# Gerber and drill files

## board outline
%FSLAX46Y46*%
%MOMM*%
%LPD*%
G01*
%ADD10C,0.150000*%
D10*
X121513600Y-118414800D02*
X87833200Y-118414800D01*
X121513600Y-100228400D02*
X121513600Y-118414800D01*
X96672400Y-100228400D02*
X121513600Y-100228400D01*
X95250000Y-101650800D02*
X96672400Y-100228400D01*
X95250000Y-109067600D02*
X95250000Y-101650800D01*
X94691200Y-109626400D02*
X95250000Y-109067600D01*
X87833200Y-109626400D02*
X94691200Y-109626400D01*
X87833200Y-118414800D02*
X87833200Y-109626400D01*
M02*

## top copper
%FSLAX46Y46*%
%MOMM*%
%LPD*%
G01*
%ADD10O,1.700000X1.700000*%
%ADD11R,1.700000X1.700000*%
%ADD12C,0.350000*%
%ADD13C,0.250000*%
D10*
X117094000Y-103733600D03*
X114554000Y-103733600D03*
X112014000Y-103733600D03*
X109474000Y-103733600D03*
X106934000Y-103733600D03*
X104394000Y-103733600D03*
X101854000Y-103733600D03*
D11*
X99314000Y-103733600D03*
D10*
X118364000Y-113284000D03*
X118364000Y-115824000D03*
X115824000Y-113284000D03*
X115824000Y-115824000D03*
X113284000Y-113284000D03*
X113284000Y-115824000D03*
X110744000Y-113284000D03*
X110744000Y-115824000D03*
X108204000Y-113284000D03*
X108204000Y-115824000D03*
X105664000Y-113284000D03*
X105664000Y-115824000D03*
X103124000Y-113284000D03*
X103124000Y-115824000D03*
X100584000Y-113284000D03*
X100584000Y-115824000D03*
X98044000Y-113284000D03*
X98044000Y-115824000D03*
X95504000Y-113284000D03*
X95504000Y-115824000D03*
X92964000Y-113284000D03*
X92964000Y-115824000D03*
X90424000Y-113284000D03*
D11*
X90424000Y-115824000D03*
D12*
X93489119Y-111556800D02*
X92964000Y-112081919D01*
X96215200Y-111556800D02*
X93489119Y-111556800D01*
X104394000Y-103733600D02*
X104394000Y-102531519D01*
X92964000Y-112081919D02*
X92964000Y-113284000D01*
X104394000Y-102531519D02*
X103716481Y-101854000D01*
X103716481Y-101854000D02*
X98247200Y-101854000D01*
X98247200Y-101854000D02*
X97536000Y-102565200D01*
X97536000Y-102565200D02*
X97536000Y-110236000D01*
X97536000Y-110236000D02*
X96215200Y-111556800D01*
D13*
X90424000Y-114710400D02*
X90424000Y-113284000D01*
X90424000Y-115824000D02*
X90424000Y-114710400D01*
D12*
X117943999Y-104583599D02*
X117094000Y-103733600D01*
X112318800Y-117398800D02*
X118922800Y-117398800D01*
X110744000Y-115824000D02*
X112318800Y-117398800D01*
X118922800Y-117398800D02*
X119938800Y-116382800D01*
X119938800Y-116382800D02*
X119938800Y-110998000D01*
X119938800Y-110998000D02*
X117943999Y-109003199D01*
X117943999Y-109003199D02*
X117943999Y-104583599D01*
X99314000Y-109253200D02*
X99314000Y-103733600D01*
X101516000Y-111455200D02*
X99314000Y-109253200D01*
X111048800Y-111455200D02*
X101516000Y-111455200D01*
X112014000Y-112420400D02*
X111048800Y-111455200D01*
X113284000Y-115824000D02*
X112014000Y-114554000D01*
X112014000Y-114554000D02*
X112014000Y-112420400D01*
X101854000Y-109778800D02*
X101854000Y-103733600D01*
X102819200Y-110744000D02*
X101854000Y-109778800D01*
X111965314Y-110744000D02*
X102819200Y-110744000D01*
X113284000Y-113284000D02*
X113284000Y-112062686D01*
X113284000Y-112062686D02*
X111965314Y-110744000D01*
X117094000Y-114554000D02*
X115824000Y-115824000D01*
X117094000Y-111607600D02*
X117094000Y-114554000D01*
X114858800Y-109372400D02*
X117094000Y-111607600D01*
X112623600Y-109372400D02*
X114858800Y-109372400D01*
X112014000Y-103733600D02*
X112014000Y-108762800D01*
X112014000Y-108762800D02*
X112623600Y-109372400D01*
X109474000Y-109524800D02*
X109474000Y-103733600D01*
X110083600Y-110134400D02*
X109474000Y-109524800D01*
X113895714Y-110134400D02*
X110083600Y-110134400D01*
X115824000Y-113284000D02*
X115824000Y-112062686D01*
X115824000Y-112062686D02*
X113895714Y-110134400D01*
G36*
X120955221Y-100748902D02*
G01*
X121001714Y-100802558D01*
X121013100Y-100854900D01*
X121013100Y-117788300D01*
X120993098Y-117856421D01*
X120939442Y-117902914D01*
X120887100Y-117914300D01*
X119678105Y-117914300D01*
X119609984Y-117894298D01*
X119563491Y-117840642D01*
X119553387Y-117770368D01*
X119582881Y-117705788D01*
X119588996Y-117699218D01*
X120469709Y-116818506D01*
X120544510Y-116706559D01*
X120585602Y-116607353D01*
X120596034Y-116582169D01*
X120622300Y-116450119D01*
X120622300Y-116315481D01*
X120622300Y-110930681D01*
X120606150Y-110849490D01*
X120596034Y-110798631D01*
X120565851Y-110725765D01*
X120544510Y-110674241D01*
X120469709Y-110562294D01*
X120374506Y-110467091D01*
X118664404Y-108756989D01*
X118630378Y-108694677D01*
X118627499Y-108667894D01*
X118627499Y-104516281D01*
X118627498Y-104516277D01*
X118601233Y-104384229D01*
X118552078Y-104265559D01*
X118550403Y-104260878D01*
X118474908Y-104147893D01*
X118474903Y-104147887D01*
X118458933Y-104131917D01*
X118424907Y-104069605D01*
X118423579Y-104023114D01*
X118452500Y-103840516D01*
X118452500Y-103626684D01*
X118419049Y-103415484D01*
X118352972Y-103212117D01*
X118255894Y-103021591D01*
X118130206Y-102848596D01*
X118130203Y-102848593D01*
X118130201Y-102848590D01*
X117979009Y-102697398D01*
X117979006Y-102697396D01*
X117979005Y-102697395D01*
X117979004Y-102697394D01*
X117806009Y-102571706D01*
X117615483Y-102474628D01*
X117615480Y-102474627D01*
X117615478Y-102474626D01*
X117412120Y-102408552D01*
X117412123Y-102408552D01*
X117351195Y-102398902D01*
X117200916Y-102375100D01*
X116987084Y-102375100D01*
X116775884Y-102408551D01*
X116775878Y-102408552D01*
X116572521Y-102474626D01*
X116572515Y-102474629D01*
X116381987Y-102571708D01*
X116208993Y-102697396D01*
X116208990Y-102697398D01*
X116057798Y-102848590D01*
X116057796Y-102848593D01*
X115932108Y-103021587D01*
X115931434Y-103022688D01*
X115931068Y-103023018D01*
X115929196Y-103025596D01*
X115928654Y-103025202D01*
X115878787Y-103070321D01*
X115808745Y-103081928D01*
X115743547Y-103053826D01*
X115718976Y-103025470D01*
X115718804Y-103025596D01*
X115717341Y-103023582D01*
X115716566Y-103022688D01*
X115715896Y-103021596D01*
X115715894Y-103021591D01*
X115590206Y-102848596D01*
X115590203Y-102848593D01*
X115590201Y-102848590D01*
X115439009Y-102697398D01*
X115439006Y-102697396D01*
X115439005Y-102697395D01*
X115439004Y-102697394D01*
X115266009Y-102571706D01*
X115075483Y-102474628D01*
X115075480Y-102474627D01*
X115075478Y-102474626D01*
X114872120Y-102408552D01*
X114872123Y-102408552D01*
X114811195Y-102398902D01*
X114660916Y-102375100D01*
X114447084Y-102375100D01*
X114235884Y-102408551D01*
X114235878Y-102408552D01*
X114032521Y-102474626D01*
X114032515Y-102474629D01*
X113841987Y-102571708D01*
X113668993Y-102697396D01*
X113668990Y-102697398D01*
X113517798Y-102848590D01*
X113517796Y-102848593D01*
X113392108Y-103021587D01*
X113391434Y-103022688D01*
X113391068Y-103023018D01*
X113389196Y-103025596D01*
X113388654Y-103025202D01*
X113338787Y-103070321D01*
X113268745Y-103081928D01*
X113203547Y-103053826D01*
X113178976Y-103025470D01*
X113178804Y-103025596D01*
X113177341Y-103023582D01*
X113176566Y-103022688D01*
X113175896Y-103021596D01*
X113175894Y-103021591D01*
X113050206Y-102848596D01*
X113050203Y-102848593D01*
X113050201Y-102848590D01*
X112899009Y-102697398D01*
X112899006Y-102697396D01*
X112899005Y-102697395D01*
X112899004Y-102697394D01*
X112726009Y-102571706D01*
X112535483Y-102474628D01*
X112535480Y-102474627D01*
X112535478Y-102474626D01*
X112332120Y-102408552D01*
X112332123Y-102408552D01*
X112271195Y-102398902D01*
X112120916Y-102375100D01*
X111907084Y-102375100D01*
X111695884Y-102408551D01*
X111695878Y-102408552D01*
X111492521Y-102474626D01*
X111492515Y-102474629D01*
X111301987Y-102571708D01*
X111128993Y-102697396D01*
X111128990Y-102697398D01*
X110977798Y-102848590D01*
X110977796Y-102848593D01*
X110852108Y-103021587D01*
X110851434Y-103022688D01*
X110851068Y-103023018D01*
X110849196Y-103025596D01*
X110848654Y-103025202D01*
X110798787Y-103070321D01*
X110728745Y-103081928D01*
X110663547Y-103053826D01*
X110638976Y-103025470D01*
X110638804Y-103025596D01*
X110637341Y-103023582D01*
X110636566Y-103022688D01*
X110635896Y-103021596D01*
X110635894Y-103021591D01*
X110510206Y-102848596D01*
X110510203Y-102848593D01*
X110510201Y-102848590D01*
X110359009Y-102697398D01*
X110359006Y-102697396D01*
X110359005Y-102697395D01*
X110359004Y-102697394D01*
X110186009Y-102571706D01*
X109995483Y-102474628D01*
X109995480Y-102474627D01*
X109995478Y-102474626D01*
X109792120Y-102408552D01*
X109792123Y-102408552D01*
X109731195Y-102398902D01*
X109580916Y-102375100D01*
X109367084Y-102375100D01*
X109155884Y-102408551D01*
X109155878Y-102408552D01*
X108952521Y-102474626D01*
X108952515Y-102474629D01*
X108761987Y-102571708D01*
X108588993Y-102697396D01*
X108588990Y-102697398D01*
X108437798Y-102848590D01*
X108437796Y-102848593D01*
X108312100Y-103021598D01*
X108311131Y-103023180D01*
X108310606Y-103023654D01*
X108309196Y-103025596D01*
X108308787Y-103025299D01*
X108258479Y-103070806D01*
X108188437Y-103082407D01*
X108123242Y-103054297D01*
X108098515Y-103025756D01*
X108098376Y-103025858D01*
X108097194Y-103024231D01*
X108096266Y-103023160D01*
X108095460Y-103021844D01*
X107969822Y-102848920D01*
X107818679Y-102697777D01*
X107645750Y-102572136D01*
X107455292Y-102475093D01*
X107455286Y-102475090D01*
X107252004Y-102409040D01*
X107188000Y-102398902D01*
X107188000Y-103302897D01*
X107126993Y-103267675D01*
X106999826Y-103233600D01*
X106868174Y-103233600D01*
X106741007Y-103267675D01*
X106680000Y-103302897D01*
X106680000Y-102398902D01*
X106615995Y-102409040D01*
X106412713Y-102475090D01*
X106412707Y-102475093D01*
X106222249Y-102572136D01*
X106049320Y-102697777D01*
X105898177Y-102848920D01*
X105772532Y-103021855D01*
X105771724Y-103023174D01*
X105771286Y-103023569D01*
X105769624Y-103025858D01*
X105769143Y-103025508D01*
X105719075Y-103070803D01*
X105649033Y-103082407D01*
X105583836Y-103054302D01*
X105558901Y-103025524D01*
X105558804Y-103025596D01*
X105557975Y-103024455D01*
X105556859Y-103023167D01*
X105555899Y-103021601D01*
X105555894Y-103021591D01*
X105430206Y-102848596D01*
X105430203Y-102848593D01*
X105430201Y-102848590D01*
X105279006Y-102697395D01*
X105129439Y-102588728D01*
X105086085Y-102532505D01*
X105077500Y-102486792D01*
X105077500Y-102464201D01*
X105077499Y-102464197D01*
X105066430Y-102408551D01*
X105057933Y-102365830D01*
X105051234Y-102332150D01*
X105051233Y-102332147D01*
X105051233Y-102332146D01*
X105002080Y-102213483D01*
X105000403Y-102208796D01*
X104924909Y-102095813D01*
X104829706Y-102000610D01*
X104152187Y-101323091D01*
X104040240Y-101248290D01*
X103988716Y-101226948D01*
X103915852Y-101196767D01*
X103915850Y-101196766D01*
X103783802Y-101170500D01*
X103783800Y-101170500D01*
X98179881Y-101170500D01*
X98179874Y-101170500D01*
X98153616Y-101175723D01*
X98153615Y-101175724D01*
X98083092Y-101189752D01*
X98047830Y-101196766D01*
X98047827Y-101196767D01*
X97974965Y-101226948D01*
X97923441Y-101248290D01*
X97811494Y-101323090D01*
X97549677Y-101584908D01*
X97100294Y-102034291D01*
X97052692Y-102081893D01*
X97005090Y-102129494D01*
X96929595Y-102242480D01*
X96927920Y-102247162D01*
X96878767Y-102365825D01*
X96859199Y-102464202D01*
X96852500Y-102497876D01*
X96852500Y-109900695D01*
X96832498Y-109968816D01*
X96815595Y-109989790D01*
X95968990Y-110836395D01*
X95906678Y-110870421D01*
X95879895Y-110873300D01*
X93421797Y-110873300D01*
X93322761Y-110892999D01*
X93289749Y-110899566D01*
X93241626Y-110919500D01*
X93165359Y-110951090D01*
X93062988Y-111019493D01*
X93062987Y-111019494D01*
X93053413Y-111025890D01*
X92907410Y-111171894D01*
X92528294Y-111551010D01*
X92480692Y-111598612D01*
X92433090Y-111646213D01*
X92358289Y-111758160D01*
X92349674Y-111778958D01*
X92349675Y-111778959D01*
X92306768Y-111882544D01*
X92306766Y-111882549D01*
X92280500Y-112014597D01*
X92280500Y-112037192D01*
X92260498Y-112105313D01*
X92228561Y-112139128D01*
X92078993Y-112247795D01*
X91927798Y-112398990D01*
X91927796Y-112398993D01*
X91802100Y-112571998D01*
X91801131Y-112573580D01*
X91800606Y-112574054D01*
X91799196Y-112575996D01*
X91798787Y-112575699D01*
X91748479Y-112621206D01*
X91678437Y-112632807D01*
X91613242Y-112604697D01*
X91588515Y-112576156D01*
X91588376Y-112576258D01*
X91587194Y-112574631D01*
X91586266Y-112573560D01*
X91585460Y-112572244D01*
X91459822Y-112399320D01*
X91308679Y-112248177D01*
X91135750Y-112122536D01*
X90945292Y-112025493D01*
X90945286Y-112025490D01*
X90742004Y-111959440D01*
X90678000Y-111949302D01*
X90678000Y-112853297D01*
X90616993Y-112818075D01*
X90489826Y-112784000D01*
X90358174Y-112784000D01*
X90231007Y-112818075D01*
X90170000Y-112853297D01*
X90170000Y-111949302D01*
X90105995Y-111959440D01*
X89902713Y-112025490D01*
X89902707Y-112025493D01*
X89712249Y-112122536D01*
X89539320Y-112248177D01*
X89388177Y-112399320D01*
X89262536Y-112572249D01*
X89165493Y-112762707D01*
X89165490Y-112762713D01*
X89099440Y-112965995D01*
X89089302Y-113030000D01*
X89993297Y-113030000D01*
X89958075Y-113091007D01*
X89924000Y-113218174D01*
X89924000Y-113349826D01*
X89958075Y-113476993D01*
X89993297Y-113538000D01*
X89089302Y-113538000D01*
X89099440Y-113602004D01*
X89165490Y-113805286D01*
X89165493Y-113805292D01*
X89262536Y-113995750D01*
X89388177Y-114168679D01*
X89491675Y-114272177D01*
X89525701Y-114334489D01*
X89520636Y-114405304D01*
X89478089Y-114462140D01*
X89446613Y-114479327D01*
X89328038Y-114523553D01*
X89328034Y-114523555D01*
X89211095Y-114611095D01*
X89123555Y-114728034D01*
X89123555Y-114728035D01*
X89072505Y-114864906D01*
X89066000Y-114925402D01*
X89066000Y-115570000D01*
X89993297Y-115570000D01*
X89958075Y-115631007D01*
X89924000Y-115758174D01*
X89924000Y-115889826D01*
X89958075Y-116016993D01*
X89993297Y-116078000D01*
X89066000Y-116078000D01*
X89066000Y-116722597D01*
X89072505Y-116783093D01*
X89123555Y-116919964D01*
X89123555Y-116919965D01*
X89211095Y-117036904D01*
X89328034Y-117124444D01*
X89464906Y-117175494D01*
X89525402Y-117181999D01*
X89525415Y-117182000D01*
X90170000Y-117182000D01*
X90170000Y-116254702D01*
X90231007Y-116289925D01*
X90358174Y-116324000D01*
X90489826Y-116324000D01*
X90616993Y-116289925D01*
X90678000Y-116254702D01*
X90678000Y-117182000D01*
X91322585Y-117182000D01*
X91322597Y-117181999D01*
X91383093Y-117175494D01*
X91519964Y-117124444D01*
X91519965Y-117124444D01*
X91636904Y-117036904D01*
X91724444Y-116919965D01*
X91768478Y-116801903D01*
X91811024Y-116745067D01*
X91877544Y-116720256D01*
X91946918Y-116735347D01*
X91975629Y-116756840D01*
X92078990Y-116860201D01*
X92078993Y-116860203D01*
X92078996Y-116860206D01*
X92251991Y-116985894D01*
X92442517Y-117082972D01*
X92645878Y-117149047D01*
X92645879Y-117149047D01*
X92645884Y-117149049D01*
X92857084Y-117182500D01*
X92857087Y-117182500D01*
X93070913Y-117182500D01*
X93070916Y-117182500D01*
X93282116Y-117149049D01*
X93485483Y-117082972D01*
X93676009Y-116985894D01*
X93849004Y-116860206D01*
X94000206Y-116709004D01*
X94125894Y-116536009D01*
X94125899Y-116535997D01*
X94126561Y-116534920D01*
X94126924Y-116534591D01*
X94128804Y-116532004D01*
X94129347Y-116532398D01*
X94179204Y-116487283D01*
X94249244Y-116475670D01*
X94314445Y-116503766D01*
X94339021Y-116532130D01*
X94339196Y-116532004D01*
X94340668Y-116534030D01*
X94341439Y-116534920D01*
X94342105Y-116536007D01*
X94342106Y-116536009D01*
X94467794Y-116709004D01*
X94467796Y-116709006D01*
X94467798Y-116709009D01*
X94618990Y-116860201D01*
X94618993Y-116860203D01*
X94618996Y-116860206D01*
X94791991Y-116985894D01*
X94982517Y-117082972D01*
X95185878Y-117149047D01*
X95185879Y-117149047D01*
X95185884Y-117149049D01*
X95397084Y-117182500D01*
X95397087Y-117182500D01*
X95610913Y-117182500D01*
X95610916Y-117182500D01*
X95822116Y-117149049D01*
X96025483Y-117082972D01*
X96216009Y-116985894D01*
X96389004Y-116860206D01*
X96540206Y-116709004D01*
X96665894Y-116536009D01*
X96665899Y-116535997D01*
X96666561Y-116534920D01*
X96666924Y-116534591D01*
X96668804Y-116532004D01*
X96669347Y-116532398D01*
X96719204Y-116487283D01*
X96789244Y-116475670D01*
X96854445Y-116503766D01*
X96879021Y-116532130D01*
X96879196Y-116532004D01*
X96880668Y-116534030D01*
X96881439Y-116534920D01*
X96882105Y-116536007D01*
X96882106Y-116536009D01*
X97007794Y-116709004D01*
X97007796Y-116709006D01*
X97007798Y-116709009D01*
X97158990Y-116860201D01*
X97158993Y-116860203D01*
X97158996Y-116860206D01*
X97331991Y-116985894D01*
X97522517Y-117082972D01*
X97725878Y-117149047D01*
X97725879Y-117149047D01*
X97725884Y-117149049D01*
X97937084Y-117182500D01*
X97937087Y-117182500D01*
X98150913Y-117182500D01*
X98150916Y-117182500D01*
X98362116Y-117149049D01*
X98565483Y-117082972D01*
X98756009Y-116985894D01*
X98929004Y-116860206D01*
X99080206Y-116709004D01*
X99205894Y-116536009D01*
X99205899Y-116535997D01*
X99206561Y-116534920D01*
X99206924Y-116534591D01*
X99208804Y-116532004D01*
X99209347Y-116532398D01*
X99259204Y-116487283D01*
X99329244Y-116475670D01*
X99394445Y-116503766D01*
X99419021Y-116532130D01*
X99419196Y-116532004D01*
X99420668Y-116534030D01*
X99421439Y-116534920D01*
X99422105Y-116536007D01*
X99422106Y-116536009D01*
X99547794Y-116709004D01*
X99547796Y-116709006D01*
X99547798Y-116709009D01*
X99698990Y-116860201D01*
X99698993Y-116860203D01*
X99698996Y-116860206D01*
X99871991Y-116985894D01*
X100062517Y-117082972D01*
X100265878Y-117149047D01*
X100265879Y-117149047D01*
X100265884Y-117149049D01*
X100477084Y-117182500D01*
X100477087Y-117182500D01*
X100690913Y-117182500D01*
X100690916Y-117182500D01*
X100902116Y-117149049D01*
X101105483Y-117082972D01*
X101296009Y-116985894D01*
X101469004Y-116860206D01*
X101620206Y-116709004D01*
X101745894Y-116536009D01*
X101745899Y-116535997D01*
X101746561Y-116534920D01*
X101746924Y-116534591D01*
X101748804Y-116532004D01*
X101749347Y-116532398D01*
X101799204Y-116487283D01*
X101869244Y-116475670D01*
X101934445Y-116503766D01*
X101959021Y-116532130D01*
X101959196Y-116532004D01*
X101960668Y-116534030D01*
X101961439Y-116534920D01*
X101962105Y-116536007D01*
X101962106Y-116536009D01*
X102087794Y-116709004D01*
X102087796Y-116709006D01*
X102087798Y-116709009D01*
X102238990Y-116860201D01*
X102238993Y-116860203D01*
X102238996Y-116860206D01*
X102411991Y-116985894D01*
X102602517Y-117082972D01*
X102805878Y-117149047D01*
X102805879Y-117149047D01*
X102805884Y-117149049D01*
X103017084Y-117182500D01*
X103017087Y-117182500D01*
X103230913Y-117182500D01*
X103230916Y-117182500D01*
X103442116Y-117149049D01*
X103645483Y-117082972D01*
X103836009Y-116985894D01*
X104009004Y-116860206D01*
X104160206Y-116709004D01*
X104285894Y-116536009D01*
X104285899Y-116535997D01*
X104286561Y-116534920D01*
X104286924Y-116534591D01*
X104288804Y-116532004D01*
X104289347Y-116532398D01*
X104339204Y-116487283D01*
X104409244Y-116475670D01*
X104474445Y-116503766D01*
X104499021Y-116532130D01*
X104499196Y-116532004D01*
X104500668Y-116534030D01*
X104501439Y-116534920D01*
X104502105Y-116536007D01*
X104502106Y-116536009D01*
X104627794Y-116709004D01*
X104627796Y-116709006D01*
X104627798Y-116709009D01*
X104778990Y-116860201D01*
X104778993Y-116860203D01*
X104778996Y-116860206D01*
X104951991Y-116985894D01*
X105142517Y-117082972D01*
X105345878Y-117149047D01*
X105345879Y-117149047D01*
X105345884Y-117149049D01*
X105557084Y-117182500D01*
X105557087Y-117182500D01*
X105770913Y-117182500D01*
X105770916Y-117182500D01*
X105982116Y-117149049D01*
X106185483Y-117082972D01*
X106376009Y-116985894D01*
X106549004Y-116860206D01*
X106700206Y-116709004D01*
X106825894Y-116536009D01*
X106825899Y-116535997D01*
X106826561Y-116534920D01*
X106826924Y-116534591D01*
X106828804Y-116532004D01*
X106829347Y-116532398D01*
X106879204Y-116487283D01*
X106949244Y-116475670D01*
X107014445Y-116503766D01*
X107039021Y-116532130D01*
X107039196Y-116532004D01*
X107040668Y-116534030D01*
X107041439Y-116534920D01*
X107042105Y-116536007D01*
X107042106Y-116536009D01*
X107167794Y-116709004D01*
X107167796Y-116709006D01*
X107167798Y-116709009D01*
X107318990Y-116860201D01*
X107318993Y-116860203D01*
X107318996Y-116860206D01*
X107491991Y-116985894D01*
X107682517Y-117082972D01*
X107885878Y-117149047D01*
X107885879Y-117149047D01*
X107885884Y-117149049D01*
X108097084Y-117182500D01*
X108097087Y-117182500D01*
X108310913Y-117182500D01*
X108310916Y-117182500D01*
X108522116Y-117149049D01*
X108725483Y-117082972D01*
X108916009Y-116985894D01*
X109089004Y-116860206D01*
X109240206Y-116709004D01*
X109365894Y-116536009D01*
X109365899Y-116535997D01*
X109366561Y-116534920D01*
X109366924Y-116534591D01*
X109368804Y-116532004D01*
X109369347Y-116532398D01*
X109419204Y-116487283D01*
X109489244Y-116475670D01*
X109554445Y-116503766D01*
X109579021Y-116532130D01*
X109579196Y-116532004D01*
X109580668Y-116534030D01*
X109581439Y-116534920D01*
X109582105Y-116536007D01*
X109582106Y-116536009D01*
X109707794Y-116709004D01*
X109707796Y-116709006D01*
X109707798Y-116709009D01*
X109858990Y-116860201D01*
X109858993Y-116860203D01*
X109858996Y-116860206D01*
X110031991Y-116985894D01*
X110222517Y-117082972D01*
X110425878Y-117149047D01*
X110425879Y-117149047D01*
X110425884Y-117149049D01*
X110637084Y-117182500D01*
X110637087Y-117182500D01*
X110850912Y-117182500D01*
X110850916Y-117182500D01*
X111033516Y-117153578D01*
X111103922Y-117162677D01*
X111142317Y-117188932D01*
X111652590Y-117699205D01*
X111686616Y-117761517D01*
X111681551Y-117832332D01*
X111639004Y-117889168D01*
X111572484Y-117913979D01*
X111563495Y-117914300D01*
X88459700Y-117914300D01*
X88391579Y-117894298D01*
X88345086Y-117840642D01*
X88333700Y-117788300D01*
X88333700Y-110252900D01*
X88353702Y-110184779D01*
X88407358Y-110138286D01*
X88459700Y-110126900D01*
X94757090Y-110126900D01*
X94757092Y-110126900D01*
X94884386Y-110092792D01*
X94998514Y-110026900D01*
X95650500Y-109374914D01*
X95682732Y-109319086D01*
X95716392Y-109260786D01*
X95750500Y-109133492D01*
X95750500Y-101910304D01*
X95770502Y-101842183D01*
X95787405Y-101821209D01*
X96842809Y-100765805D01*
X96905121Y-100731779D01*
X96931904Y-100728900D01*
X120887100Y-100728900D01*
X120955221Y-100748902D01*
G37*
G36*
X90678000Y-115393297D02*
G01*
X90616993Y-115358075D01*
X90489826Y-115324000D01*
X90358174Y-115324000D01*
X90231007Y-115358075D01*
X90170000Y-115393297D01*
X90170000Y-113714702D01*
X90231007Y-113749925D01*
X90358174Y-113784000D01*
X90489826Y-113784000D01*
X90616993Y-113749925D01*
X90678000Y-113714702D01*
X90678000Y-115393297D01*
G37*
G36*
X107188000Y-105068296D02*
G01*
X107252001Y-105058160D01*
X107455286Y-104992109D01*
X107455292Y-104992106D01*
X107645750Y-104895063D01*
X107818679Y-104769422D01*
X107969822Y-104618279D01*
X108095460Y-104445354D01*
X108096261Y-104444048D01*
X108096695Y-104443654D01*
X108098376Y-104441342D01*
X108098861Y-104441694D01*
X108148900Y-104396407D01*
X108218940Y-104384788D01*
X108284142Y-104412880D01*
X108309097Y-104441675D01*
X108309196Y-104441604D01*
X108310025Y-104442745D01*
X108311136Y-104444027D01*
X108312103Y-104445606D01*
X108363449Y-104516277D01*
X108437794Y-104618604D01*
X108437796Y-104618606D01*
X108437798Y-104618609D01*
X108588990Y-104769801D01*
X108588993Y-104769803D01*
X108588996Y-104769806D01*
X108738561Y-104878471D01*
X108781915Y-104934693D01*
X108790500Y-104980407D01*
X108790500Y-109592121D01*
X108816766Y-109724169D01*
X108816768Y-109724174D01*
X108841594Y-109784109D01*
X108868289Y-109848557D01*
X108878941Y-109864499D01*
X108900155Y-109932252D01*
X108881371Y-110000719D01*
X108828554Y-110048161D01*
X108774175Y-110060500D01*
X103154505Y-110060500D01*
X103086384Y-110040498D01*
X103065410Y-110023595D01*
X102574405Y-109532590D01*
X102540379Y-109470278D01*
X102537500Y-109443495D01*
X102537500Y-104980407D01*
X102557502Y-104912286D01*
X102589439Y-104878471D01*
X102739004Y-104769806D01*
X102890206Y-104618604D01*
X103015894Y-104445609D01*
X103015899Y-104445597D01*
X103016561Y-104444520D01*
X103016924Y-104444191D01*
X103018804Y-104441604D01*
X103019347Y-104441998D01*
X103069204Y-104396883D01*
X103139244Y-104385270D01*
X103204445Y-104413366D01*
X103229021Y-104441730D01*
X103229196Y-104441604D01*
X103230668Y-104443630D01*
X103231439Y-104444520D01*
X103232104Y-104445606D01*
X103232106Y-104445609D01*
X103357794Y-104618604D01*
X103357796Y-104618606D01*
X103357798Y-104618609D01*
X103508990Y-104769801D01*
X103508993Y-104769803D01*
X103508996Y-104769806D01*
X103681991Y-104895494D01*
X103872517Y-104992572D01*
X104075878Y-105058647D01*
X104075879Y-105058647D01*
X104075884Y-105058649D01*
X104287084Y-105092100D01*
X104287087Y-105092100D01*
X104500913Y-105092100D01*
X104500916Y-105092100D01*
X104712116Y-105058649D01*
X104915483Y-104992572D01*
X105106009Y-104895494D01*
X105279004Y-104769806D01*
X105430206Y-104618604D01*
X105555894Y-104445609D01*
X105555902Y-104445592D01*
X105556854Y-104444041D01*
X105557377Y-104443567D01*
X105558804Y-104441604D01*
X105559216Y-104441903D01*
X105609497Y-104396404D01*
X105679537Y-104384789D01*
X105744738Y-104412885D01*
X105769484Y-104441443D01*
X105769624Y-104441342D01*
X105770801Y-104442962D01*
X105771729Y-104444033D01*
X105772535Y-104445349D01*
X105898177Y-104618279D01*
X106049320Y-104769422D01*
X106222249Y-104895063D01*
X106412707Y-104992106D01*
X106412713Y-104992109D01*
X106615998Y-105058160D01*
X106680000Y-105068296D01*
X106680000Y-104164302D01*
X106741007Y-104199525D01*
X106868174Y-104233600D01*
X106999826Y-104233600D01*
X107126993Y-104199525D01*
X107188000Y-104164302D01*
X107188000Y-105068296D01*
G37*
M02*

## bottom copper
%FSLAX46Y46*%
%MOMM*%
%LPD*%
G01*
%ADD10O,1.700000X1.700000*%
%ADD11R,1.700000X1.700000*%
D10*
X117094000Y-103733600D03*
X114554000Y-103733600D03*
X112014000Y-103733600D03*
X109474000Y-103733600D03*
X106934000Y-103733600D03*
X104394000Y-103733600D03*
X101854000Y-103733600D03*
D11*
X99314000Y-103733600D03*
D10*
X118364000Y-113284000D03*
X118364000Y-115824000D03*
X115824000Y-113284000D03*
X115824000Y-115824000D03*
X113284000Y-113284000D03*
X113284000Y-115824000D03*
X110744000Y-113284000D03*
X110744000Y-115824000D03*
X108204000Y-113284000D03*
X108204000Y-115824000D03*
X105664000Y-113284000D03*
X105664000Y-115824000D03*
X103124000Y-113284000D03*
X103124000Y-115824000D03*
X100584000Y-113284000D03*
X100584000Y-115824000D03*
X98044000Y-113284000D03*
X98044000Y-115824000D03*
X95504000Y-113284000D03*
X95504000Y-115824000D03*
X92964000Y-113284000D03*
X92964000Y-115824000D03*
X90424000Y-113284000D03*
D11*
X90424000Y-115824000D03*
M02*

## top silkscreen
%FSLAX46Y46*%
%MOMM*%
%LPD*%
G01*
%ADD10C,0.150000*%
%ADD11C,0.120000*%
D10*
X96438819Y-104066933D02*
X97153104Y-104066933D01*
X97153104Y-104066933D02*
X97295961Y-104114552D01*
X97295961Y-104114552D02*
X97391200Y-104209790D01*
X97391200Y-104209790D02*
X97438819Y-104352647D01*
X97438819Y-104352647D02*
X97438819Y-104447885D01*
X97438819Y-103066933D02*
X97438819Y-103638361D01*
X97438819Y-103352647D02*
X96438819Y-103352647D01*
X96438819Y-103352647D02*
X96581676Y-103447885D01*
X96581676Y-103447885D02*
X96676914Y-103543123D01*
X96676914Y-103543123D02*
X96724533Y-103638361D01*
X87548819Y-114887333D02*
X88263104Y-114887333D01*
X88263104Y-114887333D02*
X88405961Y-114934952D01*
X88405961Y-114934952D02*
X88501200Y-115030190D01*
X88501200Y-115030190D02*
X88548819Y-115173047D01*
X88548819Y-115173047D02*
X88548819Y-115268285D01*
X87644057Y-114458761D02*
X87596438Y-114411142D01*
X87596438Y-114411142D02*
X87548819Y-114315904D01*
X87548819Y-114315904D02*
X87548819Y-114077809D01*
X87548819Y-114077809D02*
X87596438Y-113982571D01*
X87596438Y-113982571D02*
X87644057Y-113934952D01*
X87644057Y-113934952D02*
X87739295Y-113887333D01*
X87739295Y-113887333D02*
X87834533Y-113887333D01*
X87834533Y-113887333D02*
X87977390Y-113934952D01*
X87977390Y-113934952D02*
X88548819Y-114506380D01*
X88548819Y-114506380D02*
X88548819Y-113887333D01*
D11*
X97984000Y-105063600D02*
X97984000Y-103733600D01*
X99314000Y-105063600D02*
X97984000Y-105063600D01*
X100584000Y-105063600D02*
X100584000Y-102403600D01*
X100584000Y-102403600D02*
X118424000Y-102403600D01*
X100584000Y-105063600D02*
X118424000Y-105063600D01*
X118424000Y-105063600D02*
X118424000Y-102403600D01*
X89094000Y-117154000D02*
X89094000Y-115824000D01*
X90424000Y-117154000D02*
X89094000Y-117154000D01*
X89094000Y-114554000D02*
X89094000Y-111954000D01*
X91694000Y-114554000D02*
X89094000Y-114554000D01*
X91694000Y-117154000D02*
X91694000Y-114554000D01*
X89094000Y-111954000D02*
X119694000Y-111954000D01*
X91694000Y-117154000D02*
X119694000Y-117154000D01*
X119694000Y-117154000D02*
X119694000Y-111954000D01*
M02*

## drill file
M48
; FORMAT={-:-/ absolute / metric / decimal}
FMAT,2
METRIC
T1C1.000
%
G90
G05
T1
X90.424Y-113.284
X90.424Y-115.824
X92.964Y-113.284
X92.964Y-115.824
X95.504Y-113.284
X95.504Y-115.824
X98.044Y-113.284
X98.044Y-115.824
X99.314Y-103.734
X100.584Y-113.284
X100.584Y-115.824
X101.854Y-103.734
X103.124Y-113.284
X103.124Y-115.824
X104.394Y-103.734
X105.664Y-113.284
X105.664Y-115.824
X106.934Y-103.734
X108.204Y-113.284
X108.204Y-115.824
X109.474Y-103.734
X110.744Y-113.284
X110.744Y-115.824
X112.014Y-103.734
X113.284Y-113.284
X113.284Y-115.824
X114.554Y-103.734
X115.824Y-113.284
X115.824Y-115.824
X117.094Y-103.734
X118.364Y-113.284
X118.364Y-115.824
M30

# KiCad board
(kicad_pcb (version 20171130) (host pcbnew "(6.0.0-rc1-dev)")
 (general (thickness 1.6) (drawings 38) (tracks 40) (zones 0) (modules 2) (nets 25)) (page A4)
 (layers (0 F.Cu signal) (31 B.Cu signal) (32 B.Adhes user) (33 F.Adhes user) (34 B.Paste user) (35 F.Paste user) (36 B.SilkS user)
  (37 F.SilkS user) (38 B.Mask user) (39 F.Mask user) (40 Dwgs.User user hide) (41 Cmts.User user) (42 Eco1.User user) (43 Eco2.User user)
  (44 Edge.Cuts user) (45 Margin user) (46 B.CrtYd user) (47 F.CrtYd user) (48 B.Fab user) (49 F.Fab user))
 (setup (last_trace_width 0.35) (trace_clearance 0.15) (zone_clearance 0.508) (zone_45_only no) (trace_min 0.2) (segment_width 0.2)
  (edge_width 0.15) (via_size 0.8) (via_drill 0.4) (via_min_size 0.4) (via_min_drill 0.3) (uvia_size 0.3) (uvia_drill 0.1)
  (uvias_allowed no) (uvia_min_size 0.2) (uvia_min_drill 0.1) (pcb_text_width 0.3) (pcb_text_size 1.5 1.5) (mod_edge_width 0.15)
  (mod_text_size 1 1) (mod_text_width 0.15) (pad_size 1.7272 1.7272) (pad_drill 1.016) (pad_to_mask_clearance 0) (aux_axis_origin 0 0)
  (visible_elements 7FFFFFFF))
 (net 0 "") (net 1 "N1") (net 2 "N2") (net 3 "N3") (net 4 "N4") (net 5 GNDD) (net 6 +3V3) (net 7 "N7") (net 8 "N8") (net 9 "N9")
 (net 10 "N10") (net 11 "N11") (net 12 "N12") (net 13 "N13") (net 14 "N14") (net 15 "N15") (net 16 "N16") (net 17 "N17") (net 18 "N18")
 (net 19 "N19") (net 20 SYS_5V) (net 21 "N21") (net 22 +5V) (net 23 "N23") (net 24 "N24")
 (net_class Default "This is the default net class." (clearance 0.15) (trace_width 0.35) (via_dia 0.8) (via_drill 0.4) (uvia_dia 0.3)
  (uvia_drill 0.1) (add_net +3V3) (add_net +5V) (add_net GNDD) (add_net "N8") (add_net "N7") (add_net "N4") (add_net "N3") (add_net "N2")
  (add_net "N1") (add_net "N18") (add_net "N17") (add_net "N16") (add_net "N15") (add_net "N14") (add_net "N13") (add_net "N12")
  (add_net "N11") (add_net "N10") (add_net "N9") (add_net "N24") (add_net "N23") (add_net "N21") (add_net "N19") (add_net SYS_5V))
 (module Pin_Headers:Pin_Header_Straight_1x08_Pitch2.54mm (layer F.Cu) (at 99.314 103.7336 90)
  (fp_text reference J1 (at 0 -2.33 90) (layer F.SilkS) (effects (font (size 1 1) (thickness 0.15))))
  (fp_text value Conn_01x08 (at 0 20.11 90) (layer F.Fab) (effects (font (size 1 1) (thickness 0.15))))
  (fp_line (start -1.33 -1.33) (end 0 -1.33) (layer F.SilkS) (width 0.12))
  (fp_line (start -1.33 0) (end -1.33 -1.33) (layer F.SilkS) (width 0.12))
  (fp_line (start -1.33 1.27) (end 1.33 1.27) (layer F.SilkS) (width 0.12))
  (fp_line (start 1.33 1.27) (end 1.33 19.11) (layer F.SilkS) (width 0.12))
  (fp_line (start -1.33 1.27) (end -1.33 19.11) (layer F.SilkS) (width 0.12))
  (fp_line (start -1.33 19.11) (end 1.33 19.11) (layer F.SilkS) (width 0.12))
  (pad 8 thru_hole oval (at 0 17.78 90) (size 1.7 1.7) (drill 1) (layers *.Cu *.Mask) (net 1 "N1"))
  (pad 7 thru_hole oval (at 0 15.24 90) (size 1.7 1.7) (drill 1) (layers *.Cu *.Mask) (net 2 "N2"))
  (pad 6 thru_hole oval (at 0 12.7 90) (size 1.7 1.7) (drill 1) (layers *.Cu *.Mask) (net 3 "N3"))
  (pad 5 thru_hole oval (at 0 10.16 90) (size 1.7 1.7) (drill 1) (layers *.Cu *.Mask) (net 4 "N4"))
  (pad 4 thru_hole oval (at 0 7.62 90) (size 1.7 1.7) (drill 1) (layers *.Cu *.Mask) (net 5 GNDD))
  (pad 3 thru_hole oval (at 0 5.08 90) (size 1.7 1.7) (drill 1) (layers *.Cu *.Mask) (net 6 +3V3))
  (pad 2 thru_hole oval (at 0 2.54 90) (size 1.7 1.7) (drill 1) (layers *.Cu *.Mask) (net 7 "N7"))
  (pad 1 thru_hole rect (at 0 0 90) (size 1.7 1.7) (drill 1) (layers *.Cu *.Mask) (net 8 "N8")))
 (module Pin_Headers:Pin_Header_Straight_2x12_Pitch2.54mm (layer F.Cu) (at 90.424 115.824 90)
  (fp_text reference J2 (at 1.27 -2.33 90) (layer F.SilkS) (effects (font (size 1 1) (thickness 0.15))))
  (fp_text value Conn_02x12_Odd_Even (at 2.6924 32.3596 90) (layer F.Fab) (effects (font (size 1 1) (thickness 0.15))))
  (fp_line (start -1.33 -1.33) (end 0 -1.33) (layer F.SilkS) (width 0.12))
  (fp_line (start -1.33 0) (end -1.33 -1.33) (layer F.SilkS) (width 0.12))
  (fp_line (start 1.27 -1.33) (end 3.87 -1.33) (layer F.SilkS) (width 0.12))
  (fp_line (start 1.27 1.27) (end 1.27 -1.33) (layer F.SilkS) (width 0.12))
  (fp_line (start -1.33 1.27) (end 1.27 1.27) (layer F.SilkS) (width 0.12))
  (fp_line (start 3.87 -1.33) (end 3.87 29.27) (layer F.SilkS) (width 0.12))
  (fp_line (start -1.33 1.27) (end -1.33 29.27) (layer F.SilkS) (width 0.12))
  (fp_line (start -1.33 29.27) (end 3.87 29.27) (layer F.SilkS) (width 0.12))
  (pad 24 thru_hole oval (at 2.54 27.94 90) (size 1.7 1.7) (drill 1) (layers *.Cu *.Mask) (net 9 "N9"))
  (pad 23 thru_hole oval (at 0 27.94 90) (size 1.7 1.7) (drill 1) (layers *.Cu *.Mask) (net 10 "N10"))
  (pad 22 thru_hole oval (at 2.54 25.4 90) (size 1.7 1.7) (drill 1) (layers *.Cu *.Mask) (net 4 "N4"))
  (pad 21 thru_hole oval (at 0 25.4 90) (size 1.7 1.7) (drill 1) (layers *.Cu *.Mask) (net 3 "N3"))
  (pad 20 thru_hole oval (at 2.54 22.86 90) (size 1.7 1.7) (drill 1) (layers *.Cu *.Mask) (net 7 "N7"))
  (pad 19 thru_hole oval (at 0 22.86 90) (size 1.7 1.7) (drill 1) (layers *.Cu *.Mask) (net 8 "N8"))
  (pad 18 thru_hole oval (at 2.54 20.32 90) (size 1.7 1.7) (drill 1) (layers *.Cu *.Mask) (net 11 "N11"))
  (pad 17 thru_hole oval (at 0 20.32 90) (size 1.7 1.7) (drill 1) (layers *.Cu *.Mask) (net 1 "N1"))
  (pad 16 thru_hole oval (at 2.54 17.78 90) (size 1.7 1.7) (drill 1) (layers *.Cu *.Mask) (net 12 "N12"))
  (pad 15 thru_hole oval (at 0 17.78 90) (size 1.7 1.7) (drill 1) (layers *.Cu *.Mask) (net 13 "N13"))
  (pad 14 thru_hole oval (at 2.54 15.24 90) (size 1.7 1.7) (drill 1) (layers *.Cu *.Mask) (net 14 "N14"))
  (pad 13 thru_hole oval (at 0 15.24 90) (size 1.7 1.7) (drill 1) (layers *.Cu *.Mask) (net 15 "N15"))
  (pad 12 thru_hole oval (at 2.54 12.7 90) (size 1.7 1.7) (drill 1) (layers *.Cu *.Mask) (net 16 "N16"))
  (pad 11 thru_hole oval (at 0 12.7 90) (size 1.7 1.7) (drill 1) (layers *.Cu *.Mask) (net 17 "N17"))
  (pad 10 thru_hole oval (at 2.54 10.16 90) (size 1.7 1.7) (drill 1) (layers *.Cu *.Mask) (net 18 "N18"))
  (pad 9 thru_hole oval (at 0 10.16 90) (size 1.7 1.7) (drill 1) (layers *.Cu *.Mask) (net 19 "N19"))
  (pad 8 thru_hole oval (at 2.54 7.62 90) (size 1.7 1.7) (drill 1) (layers *.Cu *.Mask) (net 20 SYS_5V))
  (pad 7 thru_hole oval (at 0 7.62 90) (size 1.7 1.7) (drill 1) (layers *.Cu *.Mask) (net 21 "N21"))
  (pad 6 thru_hole oval (at 2.54 5.08 90) (size 1.7 1.7) (drill 1) (layers *.Cu *.Mask) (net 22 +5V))
  (pad 5 thru_hole oval (at 0 5.08 90) (size 1.7 1.7) (drill 1) (layers *.Cu *.Mask) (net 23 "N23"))
  (pad 4 thru_hole oval (at 2.54 2.54 90) (size 1.7 1.7) (drill 1) (layers *.Cu *.Mask) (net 6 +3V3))
  (pad 3 thru_hole oval (at 0 2.54 90) (size 1.7 1.7) (drill 1) (layers *.Cu *.Mask) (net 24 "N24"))
  (pad 2 thru_hole oval (at 2.54 0 90) (size 1.7 1.7) (drill 1) (layers *.Cu *.Mask) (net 5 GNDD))
  (pad 1 thru_hole rect (at 0 0 90) (size 1.7 1.7) (drill 1) (layers *.Cu *.Mask) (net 5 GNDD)))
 (gr_line (start 121.5136 118.4148) (end 87.8332 118.4148) (layer Edge.Cuts) (width 0.15))
 (gr_line (start 121.5136 100.2284) (end 121.5136 118.4148) (layer Edge.Cuts) (width 0.15))
 (gr_line (start 96.6724 100.2284) (end 121.5136 100.2284) (layer Edge.Cuts) (width 0.15))
 (gr_line (start 95.25 101.6508) (end 96.6724 100.2284) (layer Edge.Cuts) (width 0.15))
 (gr_line (start 95.25 109.0676) (end 95.25 101.6508) (layer Edge.Cuts) (width 0.15))
 (gr_line (start 94.6912 109.6264) (end 95.25 109.0676) (layer Edge.Cuts) (width 0.15))
 (gr_line (start 87.8332 109.6264) (end 94.6912 109.6264) (layer Edge.Cuts) (width 0.15))
 (gr_line (start 87.8332 118.4148) (end 87.8332 109.6264) (layer Edge.Cuts) (width 0.15))
 (segment (start 93.489119 111.5568) (end 92.964 112.081919) (width 0.35) (layer F.Cu) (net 6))
 (segment (start 96.2152 111.5568) (end 93.489119 111.5568) (width 0.35) (layer F.Cu) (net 6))
 (segment (start 104.394 103.7336) (end 104.394 102.531519) (width 0.35) (layer F.Cu) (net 6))
 (segment (start 92.964 112.081919) (end 92.964 113.284) (width 0.35) (layer F.Cu) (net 6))
 (segment (start 104.394 102.531519) (end 103.716481 101.854) (width 0.35) (layer F.Cu) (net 6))
 (segment (start 103.716481 101.854) (end 98.2472 101.854) (width 0.35) (layer F.Cu) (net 6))
 (segment (start 98.2472 101.854) (end 97.536 102.5652) (width 0.35) (layer F.Cu) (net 6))
 (segment (start 97.536 102.5652) (end 97.536 110.236) (width 0.35) (layer F.Cu) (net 6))
 (segment (start 97.536 110.236) (end 96.2152 111.5568) (width 0.35) (layer F.Cu) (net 6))
 (segment (start 90.424 114.7104) (end 90.424 113.284) (width 0.25) (layer F.Cu) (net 5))
 (segment (start 90.424 115.824) (end 90.424 114.7104) (width 0.25) (layer F.Cu) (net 5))
 (segment (start 117.943999 104.583599) (end 117.094 103.7336) (width 0.35) (layer F.Cu) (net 1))
 (segment (start 112.3188 117.3988) (end 118.9228 117.3988) (width 0.35) (layer F.Cu) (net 1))
 (segment (start 110.744 115.824) (end 112.3188 117.3988) (width 0.35) (layer F.Cu) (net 1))
 (segment (start 118.9228 117.3988) (end 119.9388 116.3828) (width 0.35) (layer F.Cu) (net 1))
 (segment (start 119.9388 116.3828) (end 119.9388 110.998) (width 0.35) (layer F.Cu) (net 1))
 (segment (start 119.9388 110.998) (end 117.943999 109.003199) (width 0.35) (layer F.Cu) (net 1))
 (segment (start 117.943999 109.003199) (end 117.943999 104.583599) (width 0.35) (layer F.Cu) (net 1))
 (segment (start 99.314 109.2532) (end 99.314 103.7336) (width 0.35) (layer F.Cu) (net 8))
 (segment (start 101.516 111.4552) (end 99.314 109.2532) (width 0.35) (layer F.Cu) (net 8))
 (segment (start 111.0488 111.4552) (end 101.516 111.4552) (width 0.35) (layer F.Cu) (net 8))
 (segment (start 112.014 112.4204) (end 111.0488 111.4552) (width 0.35) (layer F.Cu) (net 8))
 (segment (start 113.284 115.824) (end 112.014 114.554) (width 0.35) (layer F.Cu) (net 8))
 (segment (start 112.014 114.554) (end 112.014 112.4204) (width 0.35) (layer F.Cu) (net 8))
 (segment (start 101.854 109.7788) (end 101.854 103.7336) (width 0.35) (layer F.Cu) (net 7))
 (segment (start 102.8192 110.744) (end 101.854 109.7788) (width 0.35) (layer F.Cu) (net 7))
 (segment (start 111.965314 110.744) (end 102.8192 110.744) (width 0.35) (layer F.Cu) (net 7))
 (segment (start 113.284 113.284) (end 113.284 112.062686) (width 0.35) (layer F.Cu) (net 7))
 (segment (start 113.284 112.062686) (end 111.965314 110.744) (width 0.35) (layer F.Cu) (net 7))
 (segment (start 117.094 114.554) (end 115.824 115.824) (width 0.35) (layer F.Cu) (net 3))
 (segment (start 117.094 111.6076) (end 117.094 114.554) (width 0.35) (layer F.Cu) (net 3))
 (segment (start 114.8588 109.3724) (end 117.094 111.6076) (width 0.35) (layer F.Cu) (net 3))
 (segment (start 112.6236 109.3724) (end 114.8588 109.3724) (width 0.35) (layer F.Cu) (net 3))
 (segment (start 112.014 103.7336) (end 112.014 108.7628) (width 0.35) (layer F.Cu) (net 3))
 (segment (start 112.014 108.7628) (end 112.6236 109.3724) (width 0.35) (layer F.Cu) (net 3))
 (segment (start 109.474 109.5248) (end 109.474 103.7336) (width 0.35) (layer F.Cu) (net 4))
 (segment (start 110.0836 110.1344) (end 109.474 109.5248) (width 0.35) (layer F.Cu) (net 4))
 (segment (start 113.895714 110.1344) (end 110.0836 110.1344) (width 0.35) (layer F.Cu) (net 4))
 (segment (start 115.824 113.284) (end 115.824 112.062686) (width 0.35) (layer F.Cu) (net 4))
 (segment (start 115.824 112.062686) (end 113.895714 110.1344) (width 0.35) (layer F.Cu) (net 4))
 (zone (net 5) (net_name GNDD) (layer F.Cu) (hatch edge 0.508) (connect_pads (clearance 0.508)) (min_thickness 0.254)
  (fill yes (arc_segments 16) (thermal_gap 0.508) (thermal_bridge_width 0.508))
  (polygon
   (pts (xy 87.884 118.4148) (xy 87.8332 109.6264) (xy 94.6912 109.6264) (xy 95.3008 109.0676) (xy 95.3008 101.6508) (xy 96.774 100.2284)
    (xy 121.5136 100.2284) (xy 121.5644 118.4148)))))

